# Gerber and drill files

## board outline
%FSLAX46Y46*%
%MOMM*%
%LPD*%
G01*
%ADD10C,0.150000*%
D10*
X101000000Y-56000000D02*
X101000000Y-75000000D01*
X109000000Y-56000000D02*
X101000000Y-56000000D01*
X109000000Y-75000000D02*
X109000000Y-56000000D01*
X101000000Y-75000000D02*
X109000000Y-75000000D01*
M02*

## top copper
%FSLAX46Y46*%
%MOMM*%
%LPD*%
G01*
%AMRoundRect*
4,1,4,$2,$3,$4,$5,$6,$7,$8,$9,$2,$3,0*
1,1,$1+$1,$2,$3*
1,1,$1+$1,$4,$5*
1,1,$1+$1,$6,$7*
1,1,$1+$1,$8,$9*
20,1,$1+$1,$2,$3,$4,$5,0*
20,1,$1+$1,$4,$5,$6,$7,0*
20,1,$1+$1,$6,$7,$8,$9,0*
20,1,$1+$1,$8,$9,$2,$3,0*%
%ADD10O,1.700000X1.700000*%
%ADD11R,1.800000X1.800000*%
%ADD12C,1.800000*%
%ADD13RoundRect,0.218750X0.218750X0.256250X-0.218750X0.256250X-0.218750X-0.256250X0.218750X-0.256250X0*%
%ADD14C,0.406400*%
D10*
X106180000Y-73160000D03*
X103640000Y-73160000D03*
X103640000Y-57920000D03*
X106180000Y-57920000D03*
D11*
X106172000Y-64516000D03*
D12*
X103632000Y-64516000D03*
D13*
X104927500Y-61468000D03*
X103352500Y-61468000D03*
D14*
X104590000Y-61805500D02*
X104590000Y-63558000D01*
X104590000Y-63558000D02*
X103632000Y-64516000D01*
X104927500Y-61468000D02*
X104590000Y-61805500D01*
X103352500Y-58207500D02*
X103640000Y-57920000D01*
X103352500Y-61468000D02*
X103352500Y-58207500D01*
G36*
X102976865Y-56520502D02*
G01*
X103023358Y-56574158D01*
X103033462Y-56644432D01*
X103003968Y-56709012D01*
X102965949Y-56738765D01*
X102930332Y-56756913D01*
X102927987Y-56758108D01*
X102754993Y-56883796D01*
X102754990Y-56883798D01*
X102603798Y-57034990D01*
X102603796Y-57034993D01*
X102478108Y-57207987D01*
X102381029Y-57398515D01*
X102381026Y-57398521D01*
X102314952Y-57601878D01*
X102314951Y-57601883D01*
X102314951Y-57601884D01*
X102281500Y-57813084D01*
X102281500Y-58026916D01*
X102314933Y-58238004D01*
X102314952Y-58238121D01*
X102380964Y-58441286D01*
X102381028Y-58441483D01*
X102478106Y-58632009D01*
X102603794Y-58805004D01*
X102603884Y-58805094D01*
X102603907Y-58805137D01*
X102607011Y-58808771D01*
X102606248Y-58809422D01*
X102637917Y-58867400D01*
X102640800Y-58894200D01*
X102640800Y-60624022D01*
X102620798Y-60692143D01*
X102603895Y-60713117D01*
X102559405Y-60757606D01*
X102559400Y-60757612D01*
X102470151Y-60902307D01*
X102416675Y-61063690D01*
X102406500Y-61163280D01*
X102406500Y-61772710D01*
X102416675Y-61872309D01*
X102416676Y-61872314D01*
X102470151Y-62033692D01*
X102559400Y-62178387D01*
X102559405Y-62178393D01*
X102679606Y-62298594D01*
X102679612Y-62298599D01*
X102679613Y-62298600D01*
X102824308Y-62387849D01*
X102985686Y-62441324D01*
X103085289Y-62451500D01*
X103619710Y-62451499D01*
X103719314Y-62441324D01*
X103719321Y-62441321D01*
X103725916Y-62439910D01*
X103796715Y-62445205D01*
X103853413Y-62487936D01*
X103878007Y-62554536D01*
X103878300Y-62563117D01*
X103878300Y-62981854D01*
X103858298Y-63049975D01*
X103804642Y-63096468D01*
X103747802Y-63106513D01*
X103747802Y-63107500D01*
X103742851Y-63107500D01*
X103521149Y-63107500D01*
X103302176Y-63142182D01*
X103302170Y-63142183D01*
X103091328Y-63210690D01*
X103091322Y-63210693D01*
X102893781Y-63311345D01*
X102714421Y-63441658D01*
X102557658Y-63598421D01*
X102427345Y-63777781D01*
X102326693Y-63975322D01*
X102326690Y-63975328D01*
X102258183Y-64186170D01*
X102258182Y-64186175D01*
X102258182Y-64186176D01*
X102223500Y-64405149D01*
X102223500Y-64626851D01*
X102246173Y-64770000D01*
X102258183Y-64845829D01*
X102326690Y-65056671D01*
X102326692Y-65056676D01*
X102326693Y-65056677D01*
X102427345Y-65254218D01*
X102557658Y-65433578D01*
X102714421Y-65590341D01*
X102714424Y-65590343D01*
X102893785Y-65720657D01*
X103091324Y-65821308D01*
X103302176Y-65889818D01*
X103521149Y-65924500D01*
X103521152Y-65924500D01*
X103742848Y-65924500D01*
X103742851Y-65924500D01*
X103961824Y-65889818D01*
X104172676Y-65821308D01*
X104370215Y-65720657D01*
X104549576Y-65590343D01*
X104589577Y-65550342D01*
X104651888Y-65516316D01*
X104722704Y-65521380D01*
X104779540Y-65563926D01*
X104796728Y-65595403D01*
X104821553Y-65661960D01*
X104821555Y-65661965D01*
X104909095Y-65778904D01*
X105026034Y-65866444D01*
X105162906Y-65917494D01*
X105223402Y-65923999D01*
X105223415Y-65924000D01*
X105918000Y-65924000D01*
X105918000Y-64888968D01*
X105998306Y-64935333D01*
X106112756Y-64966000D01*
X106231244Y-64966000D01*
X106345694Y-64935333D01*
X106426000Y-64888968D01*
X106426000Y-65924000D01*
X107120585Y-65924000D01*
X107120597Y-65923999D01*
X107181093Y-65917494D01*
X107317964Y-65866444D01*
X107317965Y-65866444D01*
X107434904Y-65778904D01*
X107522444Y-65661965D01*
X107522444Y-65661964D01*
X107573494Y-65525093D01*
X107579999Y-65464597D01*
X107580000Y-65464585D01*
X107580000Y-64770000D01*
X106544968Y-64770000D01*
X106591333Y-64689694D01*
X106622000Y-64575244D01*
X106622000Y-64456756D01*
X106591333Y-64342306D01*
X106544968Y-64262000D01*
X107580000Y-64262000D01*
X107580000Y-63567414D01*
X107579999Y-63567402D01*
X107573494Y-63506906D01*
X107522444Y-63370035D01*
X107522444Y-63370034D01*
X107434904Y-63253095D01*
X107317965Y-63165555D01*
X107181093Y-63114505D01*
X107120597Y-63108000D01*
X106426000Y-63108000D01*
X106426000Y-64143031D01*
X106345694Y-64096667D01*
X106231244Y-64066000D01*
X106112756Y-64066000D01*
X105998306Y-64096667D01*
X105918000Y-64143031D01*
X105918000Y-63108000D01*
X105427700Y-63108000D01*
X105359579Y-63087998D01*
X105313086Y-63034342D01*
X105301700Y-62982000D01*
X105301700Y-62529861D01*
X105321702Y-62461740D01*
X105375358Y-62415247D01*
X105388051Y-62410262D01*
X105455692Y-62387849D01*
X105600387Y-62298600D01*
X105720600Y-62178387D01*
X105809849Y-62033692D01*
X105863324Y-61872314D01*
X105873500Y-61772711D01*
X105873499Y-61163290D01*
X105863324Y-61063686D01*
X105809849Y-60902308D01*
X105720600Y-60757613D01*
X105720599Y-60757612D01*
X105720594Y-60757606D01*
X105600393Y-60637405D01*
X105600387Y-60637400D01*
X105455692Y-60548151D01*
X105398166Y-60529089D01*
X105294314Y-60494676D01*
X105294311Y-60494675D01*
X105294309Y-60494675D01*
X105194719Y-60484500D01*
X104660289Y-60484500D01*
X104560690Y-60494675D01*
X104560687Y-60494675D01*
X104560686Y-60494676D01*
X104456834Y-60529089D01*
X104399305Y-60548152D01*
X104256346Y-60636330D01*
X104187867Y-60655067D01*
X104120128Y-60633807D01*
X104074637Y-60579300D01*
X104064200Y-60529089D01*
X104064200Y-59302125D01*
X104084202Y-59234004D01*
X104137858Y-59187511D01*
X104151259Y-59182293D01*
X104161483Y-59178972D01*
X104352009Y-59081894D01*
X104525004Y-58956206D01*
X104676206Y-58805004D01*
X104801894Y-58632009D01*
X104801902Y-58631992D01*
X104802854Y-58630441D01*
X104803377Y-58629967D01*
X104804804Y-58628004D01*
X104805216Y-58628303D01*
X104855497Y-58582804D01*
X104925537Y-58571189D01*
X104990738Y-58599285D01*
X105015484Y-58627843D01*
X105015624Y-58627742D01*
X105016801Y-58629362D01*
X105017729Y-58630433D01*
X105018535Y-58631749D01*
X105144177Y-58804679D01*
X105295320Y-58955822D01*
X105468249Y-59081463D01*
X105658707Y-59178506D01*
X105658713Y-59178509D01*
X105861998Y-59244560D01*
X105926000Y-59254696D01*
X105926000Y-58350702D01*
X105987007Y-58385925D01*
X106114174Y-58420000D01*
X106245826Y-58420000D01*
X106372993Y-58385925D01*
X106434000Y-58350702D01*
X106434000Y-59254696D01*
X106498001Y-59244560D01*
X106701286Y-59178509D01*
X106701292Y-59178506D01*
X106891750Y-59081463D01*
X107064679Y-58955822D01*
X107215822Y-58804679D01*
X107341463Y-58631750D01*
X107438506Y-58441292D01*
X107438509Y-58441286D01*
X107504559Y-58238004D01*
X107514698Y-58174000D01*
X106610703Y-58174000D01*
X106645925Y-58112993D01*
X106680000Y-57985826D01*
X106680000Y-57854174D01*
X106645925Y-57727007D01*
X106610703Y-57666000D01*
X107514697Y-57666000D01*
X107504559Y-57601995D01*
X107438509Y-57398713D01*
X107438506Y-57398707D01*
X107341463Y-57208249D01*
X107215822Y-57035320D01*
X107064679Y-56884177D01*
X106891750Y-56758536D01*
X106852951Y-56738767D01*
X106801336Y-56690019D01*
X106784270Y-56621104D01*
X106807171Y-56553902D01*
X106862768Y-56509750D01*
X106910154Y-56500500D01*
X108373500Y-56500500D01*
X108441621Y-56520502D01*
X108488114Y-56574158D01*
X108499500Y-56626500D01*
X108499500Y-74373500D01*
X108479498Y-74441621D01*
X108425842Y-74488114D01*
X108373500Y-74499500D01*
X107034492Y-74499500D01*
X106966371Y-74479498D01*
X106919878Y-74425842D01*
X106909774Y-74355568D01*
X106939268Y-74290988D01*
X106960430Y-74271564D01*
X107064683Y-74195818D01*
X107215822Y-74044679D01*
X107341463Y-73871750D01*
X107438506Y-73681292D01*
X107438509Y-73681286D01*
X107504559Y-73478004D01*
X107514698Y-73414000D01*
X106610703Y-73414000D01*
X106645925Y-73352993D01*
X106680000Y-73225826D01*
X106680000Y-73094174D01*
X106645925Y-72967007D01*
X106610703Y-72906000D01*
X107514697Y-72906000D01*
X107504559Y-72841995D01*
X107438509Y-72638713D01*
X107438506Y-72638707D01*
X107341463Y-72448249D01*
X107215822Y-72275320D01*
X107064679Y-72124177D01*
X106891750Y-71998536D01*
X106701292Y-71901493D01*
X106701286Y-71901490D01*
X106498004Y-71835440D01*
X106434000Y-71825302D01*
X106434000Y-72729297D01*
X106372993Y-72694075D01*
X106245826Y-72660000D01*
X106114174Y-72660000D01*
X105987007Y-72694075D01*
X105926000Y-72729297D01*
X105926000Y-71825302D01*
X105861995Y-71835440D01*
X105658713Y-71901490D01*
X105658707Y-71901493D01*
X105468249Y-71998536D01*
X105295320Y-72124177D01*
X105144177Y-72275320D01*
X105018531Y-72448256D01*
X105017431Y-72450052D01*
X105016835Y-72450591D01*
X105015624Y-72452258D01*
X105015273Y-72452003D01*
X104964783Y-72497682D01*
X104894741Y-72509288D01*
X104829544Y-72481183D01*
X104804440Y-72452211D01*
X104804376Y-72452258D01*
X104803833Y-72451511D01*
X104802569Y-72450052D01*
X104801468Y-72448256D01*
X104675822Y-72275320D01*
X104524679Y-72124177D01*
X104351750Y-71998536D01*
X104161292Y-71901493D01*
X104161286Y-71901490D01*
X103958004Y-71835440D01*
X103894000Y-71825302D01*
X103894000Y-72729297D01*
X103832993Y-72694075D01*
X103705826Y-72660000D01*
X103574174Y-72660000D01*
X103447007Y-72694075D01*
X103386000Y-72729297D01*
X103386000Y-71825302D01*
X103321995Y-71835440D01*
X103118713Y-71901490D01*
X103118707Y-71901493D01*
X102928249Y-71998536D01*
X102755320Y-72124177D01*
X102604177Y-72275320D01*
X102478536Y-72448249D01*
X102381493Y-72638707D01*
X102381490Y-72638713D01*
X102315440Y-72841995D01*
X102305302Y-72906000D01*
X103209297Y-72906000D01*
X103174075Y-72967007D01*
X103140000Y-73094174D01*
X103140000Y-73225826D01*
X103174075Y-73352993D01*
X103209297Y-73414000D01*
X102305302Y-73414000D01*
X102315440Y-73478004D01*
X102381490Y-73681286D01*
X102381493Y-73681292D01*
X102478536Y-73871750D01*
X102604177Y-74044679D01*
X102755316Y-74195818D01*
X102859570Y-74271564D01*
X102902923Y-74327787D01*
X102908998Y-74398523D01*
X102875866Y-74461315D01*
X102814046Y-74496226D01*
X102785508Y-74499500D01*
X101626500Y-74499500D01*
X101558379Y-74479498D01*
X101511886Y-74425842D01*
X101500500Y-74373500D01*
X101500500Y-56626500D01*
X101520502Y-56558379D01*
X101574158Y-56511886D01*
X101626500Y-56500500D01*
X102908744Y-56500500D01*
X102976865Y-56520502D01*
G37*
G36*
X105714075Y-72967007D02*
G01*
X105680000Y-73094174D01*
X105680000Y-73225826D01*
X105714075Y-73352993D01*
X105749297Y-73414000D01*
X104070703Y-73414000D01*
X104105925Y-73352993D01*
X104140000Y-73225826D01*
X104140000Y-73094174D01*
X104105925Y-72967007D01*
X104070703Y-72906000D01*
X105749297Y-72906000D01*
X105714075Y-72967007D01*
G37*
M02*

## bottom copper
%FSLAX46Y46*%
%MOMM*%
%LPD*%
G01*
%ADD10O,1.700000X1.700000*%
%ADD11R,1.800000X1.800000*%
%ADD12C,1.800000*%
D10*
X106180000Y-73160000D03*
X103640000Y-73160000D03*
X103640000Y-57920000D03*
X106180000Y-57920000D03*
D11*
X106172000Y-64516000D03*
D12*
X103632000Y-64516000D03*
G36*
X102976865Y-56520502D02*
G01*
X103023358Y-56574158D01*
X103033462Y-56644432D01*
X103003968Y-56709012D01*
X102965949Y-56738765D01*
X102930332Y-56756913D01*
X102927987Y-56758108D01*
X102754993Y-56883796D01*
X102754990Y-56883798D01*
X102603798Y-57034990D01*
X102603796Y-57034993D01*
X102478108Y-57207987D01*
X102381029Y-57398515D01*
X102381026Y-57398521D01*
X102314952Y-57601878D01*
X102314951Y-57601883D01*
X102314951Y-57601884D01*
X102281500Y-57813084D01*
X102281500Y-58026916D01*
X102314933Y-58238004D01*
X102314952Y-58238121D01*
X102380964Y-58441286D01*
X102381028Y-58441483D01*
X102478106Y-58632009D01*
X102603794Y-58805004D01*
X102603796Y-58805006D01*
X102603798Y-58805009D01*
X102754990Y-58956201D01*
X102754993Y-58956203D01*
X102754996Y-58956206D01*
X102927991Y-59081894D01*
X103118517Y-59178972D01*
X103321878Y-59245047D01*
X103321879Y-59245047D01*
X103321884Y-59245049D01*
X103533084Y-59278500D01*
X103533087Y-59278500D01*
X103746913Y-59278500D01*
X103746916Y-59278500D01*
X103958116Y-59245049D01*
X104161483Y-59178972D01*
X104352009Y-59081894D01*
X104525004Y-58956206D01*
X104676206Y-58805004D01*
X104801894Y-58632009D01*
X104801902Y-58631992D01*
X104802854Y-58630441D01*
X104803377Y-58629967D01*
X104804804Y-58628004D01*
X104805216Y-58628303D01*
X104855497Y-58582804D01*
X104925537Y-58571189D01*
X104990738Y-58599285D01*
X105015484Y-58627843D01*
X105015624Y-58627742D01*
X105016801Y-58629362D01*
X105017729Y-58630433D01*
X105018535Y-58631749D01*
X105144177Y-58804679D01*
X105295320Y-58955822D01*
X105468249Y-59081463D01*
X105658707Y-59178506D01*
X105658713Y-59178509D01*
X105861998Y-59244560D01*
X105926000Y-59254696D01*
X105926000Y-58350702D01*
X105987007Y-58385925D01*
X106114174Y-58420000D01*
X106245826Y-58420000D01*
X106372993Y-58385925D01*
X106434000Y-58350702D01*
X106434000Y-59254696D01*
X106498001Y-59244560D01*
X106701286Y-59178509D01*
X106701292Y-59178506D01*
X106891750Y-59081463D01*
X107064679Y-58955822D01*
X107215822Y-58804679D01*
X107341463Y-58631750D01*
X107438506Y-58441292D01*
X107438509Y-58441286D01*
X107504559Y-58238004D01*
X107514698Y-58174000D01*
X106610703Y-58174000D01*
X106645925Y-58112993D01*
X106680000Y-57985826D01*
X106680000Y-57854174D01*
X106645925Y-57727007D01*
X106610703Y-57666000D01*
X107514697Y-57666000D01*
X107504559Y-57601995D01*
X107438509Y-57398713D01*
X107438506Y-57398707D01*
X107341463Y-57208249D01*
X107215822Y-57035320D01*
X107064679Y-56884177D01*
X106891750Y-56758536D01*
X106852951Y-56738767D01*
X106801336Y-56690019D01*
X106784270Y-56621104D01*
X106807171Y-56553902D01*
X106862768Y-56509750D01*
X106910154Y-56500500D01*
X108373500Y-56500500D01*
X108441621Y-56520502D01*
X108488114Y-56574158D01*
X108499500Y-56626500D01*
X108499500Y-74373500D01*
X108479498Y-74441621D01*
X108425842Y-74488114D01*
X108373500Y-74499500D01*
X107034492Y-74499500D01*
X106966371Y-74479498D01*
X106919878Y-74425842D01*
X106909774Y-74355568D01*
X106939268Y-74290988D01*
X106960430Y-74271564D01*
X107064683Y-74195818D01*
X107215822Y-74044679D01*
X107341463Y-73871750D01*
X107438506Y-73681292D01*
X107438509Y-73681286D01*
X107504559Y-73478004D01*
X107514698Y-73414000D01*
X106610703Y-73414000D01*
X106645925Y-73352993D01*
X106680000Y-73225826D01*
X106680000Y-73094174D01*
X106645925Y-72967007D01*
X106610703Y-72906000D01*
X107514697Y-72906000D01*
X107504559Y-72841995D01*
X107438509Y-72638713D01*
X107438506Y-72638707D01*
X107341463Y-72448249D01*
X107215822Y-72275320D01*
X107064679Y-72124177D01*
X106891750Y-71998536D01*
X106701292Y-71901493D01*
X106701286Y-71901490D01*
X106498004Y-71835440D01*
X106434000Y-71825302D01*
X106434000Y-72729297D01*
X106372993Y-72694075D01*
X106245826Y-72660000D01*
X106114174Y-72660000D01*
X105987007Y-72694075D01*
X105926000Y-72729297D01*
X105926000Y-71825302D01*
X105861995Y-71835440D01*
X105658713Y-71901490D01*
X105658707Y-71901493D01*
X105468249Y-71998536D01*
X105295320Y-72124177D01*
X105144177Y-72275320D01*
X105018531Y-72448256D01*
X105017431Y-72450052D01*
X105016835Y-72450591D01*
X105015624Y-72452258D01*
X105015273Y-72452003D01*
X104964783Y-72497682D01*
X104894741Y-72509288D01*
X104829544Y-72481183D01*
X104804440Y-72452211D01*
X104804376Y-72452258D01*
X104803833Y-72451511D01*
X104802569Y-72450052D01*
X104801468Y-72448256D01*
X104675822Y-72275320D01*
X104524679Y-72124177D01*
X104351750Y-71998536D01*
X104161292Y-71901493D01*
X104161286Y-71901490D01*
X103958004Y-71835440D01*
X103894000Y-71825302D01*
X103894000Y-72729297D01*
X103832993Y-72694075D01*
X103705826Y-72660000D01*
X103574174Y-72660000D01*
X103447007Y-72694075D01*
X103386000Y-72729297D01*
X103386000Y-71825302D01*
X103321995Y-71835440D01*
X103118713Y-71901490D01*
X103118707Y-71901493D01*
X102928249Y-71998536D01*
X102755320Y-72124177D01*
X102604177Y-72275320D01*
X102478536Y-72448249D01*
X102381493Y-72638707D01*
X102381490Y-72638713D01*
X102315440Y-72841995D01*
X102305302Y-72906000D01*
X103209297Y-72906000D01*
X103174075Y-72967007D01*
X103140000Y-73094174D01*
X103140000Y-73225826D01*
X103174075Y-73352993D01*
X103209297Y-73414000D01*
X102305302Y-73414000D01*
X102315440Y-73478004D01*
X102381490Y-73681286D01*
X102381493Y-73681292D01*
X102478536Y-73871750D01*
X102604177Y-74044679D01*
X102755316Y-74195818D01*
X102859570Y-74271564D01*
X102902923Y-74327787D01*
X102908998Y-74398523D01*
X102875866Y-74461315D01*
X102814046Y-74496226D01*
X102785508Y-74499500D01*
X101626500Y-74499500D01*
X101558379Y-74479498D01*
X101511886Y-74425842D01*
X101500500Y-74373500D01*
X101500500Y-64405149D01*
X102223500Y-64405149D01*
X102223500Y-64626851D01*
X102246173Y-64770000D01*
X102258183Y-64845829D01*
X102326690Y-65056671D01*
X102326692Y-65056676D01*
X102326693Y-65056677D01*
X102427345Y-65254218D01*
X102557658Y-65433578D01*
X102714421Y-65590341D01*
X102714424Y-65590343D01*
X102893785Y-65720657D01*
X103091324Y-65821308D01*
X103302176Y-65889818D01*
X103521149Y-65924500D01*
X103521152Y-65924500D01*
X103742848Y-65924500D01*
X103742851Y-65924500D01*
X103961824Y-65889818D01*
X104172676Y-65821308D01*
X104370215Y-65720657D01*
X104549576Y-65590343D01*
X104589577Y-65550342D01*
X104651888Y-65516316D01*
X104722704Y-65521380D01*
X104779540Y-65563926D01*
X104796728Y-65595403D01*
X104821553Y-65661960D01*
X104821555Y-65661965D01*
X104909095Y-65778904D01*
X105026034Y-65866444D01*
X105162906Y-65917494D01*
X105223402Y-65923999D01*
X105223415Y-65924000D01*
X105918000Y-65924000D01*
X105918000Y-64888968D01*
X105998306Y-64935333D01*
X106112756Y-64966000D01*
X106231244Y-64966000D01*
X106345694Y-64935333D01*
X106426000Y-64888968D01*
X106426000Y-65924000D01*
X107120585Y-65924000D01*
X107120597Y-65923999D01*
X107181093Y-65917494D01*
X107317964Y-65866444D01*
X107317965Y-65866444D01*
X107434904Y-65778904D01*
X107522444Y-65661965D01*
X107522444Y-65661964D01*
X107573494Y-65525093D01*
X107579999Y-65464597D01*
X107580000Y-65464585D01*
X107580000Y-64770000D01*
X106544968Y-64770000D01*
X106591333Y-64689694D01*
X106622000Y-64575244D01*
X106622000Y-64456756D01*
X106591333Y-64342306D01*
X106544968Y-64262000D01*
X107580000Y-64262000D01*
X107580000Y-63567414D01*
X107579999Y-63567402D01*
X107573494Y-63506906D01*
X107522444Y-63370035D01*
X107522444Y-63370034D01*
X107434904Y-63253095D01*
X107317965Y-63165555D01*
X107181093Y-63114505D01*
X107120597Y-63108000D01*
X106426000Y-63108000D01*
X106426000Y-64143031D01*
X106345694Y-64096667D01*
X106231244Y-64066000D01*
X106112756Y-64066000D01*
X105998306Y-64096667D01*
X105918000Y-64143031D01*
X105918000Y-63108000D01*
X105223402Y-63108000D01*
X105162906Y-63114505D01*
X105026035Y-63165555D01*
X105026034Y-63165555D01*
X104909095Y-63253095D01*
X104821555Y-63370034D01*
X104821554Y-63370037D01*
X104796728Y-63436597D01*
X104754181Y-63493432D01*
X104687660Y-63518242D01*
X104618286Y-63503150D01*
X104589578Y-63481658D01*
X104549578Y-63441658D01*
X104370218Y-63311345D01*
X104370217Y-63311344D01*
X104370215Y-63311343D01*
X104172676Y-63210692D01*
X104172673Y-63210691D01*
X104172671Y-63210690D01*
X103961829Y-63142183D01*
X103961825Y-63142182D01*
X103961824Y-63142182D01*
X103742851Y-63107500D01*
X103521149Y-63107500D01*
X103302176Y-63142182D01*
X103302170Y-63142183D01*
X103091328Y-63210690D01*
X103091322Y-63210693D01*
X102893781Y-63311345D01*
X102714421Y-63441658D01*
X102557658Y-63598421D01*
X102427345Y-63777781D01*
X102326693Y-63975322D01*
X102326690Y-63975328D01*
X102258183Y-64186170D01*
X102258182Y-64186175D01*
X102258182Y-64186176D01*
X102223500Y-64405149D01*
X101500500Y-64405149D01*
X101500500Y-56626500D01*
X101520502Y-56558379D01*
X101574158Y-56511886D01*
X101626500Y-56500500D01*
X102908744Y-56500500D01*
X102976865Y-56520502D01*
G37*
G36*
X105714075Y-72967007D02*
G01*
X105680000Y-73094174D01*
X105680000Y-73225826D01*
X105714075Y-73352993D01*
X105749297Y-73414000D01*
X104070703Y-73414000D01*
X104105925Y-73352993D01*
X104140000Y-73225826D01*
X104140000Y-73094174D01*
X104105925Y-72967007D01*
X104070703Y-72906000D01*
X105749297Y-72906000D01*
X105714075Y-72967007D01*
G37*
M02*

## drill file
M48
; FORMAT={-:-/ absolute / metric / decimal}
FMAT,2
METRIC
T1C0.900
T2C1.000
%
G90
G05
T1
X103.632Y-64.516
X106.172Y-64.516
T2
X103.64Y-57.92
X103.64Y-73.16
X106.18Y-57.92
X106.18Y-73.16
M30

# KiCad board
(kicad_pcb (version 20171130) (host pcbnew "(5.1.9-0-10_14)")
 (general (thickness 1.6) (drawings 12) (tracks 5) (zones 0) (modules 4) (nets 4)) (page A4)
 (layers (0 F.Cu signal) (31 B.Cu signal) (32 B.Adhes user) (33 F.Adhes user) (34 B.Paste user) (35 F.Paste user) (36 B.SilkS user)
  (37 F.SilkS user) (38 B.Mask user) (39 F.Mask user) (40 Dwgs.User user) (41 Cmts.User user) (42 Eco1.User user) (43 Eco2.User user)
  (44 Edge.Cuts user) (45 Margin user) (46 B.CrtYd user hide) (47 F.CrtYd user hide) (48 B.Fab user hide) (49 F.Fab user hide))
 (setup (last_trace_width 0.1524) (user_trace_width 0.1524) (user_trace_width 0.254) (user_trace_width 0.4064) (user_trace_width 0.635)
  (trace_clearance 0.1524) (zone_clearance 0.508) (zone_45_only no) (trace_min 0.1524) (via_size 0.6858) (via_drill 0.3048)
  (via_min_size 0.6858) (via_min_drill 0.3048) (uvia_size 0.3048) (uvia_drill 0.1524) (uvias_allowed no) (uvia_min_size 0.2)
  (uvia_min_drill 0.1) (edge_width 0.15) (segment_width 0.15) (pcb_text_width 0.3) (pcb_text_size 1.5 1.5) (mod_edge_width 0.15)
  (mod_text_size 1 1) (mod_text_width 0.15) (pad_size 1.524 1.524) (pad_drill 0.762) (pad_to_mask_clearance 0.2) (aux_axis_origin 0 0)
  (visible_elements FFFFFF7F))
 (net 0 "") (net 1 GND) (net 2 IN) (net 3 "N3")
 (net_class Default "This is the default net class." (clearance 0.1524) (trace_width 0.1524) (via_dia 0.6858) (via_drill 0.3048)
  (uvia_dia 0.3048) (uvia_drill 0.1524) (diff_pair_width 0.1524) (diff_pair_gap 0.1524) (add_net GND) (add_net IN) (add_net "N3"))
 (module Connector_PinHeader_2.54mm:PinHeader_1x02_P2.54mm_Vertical (layer B.Cu) (at 103.64 73.16 270)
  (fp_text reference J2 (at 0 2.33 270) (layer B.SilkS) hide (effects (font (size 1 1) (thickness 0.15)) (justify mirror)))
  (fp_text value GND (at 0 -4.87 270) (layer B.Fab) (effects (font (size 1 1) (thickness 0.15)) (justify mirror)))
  (pad 2 thru_hole oval (at 0 -2.54 270) (size 1.7 1.7) (drill 1) (layers *.Cu *.Mask) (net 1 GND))
  (pad 1 thru_hole oval (at 0 0 270) (size 1.7 1.7) (drill 1) (layers *.Cu *.Mask) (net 1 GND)))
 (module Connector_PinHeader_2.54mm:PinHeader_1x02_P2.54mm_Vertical (layer B.Cu) (at 103.64 57.92 270)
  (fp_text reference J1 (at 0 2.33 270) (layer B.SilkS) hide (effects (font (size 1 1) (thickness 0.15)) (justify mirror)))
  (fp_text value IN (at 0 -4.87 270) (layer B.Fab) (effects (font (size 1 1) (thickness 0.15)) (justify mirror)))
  (pad 1 thru_hole oval (at 0 0 270) (size 1.7 1.7) (drill 1) (layers *.Cu *.Mask) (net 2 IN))
  (pad 2 thru_hole oval (at 0 -2.54 270) (size 1.7 1.7) (drill 1) (layers *.Cu *.Mask) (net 1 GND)))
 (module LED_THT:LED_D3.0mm (layer F.Cu) (at 106.172 64.516 180)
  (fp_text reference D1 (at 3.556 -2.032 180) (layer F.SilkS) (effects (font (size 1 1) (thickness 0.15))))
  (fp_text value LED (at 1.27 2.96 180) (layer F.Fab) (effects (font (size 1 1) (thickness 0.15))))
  (pad 1 thru_hole rect (at 0 0 180) (size 1.8 1.8) (drill 0.9) (layers *.Cu *.Mask) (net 1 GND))
  (pad 2 thru_hole circle (at 2.54 0 180) (size 1.8 1.8) (drill 0.9) (layers *.Cu *.Mask) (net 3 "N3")))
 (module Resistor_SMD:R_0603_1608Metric (layer F.Cu) (at 104.14 61.468 180)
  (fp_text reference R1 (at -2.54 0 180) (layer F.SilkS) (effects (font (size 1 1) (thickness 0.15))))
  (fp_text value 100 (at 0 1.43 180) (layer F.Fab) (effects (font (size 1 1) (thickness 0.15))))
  (pad 1 smd roundrect (at -0.7875 0 180) (size 0.875 0.95) (layers F.Cu F.Paste F.Mask) (roundrect_rratio 0.25) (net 3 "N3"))
  (pad 2 smd roundrect (at 0.7875 0 180) (size 0.875 0.95) (layers F.Cu F.Paste F.Mask) (roundrect_rratio 0.25) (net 2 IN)))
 (gr_line (start 101 56) (end 101 75) (layer Edge.Cuts) (width 0.15))
 (gr_line (start 109 56) (end 101 56) (layer Edge.Cuts) (width 0.15))
 (gr_line (start 109 75) (end 109 56) (layer Edge.Cuts) (width 0.15))
 (gr_line (start 101 75) (end 109 75) (layer Edge.Cuts) (width 0.15))
 (segment (start 104.59 61.8055) (end 104.59 63.558) (width 0.4064) (layer F.Cu) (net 3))
 (segment (start 104.59 63.558) (end 103.632 64.516) (width 0.4064) (layer F.Cu) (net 3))
 (segment (start 104.9275 61.468) (end 104.59 61.8055) (width 0.4064) (layer F.Cu) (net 3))
 (segment (start 103.3525 58.2075) (end 103.64 57.92) (width 0.4064) (layer F.Cu) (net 2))
 (segment (start 103.3525 61.468) (end 103.3525 58.2075) (width 0.4064) (layer F.Cu) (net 2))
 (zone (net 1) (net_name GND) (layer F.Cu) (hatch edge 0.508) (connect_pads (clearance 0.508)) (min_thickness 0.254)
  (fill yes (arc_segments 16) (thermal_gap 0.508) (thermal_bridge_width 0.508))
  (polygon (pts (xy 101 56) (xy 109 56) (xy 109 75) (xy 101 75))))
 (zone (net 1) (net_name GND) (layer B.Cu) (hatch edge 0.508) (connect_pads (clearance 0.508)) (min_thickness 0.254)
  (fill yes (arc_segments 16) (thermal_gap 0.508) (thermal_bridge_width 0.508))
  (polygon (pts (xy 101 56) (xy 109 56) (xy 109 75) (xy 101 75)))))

